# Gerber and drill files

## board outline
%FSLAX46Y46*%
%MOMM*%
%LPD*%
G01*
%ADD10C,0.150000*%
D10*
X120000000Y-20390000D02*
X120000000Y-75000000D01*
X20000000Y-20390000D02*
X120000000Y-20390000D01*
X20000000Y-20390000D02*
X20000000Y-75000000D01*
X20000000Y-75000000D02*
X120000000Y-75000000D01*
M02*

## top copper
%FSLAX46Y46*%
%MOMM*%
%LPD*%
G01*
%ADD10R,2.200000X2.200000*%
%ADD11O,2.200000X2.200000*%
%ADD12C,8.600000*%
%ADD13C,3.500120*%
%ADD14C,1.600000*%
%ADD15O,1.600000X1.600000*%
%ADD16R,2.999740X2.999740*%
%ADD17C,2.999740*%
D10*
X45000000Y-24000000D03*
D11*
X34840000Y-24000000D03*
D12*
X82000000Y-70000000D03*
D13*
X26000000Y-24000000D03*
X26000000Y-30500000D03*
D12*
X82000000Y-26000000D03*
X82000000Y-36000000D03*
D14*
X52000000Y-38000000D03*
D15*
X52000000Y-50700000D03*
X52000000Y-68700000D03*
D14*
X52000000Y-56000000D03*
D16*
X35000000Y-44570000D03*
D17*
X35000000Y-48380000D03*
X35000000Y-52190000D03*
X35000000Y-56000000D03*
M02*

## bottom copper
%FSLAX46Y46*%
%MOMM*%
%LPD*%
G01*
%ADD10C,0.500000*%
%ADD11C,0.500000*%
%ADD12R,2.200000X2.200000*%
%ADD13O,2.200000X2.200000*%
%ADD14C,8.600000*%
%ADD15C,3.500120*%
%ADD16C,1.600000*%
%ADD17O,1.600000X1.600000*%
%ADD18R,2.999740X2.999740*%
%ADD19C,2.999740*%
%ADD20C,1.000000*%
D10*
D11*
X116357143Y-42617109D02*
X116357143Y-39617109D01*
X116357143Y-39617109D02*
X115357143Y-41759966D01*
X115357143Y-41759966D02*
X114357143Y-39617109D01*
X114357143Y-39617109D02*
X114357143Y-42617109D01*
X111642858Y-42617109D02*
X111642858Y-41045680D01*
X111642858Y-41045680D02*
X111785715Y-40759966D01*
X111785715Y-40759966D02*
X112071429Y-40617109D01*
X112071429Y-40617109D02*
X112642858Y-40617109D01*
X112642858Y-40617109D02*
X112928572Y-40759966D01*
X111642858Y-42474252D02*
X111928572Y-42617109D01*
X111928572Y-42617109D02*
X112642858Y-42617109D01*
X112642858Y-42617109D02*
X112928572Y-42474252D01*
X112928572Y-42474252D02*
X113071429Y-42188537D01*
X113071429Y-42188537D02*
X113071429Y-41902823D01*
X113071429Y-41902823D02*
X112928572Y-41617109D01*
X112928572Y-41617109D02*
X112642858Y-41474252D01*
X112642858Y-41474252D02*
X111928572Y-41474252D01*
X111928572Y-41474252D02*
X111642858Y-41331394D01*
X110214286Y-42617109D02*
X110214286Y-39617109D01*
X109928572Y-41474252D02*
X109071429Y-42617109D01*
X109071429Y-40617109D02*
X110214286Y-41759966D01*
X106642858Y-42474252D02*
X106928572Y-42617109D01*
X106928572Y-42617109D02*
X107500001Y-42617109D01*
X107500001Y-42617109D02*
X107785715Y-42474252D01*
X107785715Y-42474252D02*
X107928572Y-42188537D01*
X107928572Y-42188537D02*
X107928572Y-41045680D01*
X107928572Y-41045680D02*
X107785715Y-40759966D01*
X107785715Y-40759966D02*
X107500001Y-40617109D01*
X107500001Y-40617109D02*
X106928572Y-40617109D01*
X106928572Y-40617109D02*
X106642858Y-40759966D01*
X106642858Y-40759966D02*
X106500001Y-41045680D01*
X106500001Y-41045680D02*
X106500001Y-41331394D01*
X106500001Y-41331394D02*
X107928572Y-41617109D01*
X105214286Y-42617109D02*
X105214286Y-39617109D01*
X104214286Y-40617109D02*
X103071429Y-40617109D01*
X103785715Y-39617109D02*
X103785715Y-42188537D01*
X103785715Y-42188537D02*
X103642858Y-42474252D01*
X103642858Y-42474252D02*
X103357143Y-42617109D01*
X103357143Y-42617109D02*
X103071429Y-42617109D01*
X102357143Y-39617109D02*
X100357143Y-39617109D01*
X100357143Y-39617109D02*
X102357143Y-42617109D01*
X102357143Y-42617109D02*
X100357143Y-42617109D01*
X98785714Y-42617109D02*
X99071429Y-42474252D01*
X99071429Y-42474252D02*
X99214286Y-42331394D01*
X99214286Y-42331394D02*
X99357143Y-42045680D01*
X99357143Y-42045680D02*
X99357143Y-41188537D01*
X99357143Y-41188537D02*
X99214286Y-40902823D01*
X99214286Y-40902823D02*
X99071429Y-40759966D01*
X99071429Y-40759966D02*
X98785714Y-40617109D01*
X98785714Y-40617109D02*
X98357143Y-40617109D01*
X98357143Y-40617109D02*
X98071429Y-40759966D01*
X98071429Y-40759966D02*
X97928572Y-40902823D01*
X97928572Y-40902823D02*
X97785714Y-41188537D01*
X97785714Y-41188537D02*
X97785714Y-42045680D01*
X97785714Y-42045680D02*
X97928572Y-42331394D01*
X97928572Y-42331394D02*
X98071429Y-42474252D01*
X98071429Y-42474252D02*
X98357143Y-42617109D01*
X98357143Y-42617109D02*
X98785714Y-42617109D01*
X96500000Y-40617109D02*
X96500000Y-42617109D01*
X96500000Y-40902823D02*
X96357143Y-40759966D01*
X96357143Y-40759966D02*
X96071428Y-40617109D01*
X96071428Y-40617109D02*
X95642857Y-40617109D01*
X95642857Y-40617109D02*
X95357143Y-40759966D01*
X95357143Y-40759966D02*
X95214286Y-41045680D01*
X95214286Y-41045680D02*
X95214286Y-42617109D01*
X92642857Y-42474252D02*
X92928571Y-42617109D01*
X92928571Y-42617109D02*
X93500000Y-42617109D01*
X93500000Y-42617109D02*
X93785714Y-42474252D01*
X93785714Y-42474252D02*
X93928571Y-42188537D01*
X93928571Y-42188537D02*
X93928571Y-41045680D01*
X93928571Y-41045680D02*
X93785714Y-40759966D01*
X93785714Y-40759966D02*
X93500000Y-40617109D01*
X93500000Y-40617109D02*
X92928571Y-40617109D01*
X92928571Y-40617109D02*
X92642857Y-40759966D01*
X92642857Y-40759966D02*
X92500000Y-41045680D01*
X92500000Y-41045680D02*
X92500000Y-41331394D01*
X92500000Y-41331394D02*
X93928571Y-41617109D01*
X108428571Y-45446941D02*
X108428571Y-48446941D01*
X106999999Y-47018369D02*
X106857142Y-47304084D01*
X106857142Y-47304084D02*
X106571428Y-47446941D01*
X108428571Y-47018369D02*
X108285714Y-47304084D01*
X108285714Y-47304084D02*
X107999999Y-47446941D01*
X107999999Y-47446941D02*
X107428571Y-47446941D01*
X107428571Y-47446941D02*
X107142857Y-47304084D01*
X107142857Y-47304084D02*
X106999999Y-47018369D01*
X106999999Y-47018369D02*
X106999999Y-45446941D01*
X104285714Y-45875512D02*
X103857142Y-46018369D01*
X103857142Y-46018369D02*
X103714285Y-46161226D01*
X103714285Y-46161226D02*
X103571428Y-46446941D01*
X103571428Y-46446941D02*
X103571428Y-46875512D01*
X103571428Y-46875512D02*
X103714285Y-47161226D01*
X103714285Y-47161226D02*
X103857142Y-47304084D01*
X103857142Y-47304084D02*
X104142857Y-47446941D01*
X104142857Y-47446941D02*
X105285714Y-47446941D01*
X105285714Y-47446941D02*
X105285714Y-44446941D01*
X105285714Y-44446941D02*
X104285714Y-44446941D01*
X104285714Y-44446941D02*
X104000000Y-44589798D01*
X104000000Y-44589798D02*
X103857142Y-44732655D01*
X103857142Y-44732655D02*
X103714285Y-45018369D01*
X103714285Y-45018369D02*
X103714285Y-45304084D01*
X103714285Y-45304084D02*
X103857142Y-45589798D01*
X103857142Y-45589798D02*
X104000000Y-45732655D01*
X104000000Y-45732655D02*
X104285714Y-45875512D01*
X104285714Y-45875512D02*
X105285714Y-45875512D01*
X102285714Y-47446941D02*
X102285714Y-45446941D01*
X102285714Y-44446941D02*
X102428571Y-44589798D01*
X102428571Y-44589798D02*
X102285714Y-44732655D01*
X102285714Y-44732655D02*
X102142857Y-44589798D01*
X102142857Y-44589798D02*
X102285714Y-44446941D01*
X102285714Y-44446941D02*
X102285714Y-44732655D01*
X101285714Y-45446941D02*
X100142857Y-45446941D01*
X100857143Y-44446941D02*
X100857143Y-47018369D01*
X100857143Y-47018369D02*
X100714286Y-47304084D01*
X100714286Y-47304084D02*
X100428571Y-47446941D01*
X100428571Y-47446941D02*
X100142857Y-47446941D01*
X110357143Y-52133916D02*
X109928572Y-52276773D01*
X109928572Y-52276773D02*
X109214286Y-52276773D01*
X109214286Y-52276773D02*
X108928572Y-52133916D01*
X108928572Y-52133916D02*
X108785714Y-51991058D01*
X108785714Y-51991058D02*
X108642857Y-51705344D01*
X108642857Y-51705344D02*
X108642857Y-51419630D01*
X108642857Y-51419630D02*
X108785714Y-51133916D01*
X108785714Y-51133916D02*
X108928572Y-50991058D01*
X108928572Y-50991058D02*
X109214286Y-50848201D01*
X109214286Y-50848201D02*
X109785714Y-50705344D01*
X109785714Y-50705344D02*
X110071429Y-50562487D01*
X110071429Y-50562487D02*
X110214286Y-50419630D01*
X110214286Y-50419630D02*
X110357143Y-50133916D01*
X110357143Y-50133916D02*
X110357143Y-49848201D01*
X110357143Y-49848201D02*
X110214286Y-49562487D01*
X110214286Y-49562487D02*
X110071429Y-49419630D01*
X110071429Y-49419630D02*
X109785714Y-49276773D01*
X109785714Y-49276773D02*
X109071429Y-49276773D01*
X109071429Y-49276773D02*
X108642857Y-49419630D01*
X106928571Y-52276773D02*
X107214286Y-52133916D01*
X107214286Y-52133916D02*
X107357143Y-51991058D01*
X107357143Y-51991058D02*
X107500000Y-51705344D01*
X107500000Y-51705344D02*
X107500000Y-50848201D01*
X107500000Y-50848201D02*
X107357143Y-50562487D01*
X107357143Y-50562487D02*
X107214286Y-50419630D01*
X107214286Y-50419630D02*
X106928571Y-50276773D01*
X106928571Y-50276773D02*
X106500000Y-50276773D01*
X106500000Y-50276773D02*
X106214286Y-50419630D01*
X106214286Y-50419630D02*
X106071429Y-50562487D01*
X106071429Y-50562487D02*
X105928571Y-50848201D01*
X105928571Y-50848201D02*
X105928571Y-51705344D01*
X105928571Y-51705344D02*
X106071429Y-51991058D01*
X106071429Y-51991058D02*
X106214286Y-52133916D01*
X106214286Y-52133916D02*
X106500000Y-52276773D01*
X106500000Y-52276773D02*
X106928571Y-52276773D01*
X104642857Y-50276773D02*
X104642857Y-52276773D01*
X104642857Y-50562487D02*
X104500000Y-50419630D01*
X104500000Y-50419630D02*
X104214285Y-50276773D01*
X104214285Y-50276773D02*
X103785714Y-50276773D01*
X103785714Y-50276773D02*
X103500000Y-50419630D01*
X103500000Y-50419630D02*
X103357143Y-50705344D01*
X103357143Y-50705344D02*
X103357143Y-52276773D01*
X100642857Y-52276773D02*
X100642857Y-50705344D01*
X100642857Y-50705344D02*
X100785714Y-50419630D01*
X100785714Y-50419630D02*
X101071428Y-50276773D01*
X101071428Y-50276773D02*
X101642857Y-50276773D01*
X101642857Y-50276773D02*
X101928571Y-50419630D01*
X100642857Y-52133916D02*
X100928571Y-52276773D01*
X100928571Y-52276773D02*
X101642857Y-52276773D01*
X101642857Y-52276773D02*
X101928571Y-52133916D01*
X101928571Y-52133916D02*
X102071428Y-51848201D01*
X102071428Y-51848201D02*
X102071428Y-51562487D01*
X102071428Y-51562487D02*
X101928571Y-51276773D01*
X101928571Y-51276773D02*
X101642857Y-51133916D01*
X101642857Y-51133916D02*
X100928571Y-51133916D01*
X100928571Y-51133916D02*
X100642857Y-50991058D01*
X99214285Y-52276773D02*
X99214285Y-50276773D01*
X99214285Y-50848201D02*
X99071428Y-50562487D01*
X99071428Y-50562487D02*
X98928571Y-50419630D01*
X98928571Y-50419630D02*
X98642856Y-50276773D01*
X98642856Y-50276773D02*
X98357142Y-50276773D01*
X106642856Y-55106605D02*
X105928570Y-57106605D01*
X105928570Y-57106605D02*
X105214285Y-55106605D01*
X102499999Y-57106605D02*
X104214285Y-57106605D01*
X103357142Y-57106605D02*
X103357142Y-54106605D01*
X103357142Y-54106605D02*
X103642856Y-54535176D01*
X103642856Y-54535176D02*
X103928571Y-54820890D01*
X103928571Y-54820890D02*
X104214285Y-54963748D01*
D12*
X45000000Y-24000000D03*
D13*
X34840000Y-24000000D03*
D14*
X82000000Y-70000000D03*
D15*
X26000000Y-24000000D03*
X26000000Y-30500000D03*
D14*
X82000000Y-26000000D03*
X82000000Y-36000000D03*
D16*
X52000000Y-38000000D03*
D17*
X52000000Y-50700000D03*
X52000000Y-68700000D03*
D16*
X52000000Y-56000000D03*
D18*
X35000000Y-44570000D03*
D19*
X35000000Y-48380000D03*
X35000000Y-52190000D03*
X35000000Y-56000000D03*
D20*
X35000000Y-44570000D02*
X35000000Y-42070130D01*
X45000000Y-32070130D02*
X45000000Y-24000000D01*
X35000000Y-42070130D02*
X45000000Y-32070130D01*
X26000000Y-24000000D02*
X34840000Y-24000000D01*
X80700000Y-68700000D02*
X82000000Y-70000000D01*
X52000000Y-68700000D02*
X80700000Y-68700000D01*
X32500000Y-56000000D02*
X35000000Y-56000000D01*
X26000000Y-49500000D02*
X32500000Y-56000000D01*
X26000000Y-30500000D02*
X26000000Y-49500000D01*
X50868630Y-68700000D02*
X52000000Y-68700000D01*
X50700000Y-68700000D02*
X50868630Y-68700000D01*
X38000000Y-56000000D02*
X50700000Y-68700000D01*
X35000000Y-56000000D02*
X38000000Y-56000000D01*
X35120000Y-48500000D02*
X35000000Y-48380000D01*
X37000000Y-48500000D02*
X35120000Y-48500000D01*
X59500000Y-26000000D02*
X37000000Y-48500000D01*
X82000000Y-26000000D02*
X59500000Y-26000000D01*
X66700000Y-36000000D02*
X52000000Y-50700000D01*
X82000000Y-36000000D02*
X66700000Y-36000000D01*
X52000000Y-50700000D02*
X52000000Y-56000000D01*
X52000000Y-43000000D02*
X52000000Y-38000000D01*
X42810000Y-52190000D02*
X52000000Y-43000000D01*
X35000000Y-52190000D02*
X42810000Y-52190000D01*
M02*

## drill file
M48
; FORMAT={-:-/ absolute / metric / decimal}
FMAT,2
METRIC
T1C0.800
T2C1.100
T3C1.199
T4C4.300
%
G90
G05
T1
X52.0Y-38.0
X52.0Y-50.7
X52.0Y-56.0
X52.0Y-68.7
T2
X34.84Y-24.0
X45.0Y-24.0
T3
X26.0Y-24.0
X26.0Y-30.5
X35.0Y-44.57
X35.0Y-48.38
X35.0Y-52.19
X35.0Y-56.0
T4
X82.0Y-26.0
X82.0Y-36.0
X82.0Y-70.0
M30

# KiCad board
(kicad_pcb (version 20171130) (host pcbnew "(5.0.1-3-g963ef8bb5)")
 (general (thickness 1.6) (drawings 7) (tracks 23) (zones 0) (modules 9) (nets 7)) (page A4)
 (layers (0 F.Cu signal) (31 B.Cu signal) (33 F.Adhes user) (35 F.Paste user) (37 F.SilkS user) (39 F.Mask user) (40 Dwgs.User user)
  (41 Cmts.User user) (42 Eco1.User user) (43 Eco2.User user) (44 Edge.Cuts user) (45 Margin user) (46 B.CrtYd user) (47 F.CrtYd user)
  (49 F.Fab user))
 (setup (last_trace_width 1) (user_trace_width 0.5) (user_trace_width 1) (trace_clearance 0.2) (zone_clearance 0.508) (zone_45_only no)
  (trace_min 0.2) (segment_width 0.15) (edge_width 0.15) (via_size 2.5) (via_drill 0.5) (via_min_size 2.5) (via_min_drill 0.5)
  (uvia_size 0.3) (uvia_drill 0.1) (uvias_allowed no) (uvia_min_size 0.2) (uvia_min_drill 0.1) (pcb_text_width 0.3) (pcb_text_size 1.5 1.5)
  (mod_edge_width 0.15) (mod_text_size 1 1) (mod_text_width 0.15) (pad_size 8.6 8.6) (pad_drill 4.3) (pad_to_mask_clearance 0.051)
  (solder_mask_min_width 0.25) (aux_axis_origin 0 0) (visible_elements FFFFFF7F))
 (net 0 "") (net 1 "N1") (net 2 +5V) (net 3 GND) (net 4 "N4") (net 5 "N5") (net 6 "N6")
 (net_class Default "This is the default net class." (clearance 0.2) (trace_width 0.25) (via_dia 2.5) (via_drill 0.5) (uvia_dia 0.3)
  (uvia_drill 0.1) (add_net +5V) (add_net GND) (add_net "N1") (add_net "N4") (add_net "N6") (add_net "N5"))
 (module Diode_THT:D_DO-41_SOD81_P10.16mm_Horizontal (layer F.Cu) (at 45 24 180)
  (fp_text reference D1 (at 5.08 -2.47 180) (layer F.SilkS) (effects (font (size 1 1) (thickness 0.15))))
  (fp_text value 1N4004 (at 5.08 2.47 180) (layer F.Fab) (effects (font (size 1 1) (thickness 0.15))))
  (pad 1 thru_hole rect (at 0 0 180) (size 2.2 2.2) (drill 1.1) (layers *.Cu *.Mask) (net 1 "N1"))
  (pad 2 thru_hole oval (at 10.16 0 180) (size 2.2 2.2) (drill 1.1) (layers *.Cu *.Mask) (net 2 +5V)))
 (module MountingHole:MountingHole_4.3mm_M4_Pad (layer F.Cu) (at 82 70)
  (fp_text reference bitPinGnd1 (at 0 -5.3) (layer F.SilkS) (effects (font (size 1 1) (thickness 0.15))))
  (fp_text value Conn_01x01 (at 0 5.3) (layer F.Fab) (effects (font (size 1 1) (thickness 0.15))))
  (pad 1 thru_hole circle (at 0 0) (size 8.6 8.6) (drill 4.3) (layers *.Cu *.Mask) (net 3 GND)))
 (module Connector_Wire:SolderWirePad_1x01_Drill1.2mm (layer F.Cu) (at 26 24 270)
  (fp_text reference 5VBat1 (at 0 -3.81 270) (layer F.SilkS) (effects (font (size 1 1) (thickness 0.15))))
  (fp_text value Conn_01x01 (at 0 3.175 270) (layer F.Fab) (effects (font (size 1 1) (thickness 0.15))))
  (pad 1 thru_hole circle (at 0 0 270) (size 3.50012 3.50012) (drill 1.19888) (layers *.Cu *.Mask) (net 2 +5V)))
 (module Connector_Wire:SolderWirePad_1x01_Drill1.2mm (layer F.Cu) (at 26 30.5 270)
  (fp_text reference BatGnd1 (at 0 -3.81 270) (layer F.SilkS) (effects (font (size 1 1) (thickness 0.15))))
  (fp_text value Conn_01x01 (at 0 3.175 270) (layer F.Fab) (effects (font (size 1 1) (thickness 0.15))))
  (pad 1 thru_hole circle (at 0 0 270) (size 3.50012 3.50012) (drill 1.19888) (layers *.Cu *.Mask) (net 3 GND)))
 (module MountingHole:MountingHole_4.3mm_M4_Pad (layer F.Cu) (at 82 26)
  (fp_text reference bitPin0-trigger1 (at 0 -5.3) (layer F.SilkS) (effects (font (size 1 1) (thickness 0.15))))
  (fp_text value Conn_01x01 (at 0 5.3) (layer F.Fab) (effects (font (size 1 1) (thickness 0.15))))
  (pad 1 thru_hole circle (at 0 0) (size 8.6 8.6) (drill 4.3) (layers *.Cu *.Mask) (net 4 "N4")))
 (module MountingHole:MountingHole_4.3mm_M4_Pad (layer F.Cu) (at 82 36)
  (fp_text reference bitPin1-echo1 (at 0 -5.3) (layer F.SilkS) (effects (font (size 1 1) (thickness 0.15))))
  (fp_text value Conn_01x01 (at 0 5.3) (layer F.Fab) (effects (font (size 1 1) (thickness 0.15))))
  (pad 1 thru_hole circle (at 0 0) (size 8.6 8.6) (drill 4.3) (layers *.Cu *.Mask) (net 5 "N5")))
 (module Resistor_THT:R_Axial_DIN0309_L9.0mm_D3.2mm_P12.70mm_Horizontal (layer F.Cu) (at 52 38 270)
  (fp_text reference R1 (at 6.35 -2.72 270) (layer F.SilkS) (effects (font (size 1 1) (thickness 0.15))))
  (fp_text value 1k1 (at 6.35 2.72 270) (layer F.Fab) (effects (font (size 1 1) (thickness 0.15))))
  (pad 1 thru_hole circle (at 0 0 270) (size 1.6 1.6) (drill 0.8) (layers *.Cu *.Mask) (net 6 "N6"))
  (pad 2 thru_hole oval (at 12.7 0 270) (size 1.6 1.6) (drill 0.8) (layers *.Cu *.Mask) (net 5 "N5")))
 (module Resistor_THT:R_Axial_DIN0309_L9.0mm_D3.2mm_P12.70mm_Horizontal (layer F.Cu) (at 52 56 270)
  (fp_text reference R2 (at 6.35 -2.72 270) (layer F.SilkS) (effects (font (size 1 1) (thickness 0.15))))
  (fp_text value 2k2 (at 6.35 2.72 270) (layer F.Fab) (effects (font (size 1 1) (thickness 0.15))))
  (pad 2 thru_hole oval (at 12.7 0 270) (size 1.6 1.6) (drill 0.8) (layers *.Cu *.Mask) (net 3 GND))
  (pad 1 thru_hole circle (at 0 0 270) (size 1.6 1.6) (drill 0.8) (layers *.Cu *.Mask) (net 5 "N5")))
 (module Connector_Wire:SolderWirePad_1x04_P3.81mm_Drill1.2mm (layer F.Cu) (at 35 44.57 270)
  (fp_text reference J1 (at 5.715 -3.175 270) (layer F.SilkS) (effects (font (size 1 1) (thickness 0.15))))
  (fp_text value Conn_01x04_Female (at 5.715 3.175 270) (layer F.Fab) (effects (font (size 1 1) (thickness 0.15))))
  (pad 1 thru_hole rect (at 0 0 270) (size 2.99974 2.99974) (drill 1.19888) (layers *.Cu *.Mask) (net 1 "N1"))
  (pad 2 thru_hole circle (at 3.81 0 270) (size 2.99974 2.99974) (drill 1.19888) (layers *.Cu *.Mask) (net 4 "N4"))
  (pad 3 thru_hole circle (at 7.62 0 270) (size 2.99974 2.99974) (drill 1.19888) (layers *.Cu *.Mask) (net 6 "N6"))
  (pad 4 thru_hole circle (at 11.43 0 270) (size 2.99974 2.99974) (drill 1.19888) (layers *.Cu *.Mask) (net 3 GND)))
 (gr_line (start 120 20.39) (end 120 75) (layer Edge.Cuts) (width 0.15))
 (gr_line (start 20 20.39) (end 120 20.39) (layer Edge.Cuts) (width 0.15))
 (gr_line (start 20 20.39) (end 20 75) (layer Edge.Cuts) (width 0.15))
 (gr_line (start 20 75) (end 120 75) (layer Edge.Cuts) (width 0.15))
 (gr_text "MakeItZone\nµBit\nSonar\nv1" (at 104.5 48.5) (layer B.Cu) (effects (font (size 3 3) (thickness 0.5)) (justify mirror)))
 (segment (start 35 44.57) (end 35 42.07013) (width 1) (layer B.Cu) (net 1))
 (segment (start 45 32.07013) (end 45 24) (width 1) (layer B.Cu) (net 1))
 (segment (start 35 42.07013) (end 45 32.07013) (width 1) (layer B.Cu) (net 1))
 (segment (start 26 24) (end 34.84 24) (width 1) (layer B.Cu) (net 2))
 (segment (start 80.7 68.7) (end 82 70) (width 1) (layer B.Cu) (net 3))
 (segment (start 52 68.7) (end 80.7 68.7) (width 1) (layer B.Cu) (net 3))
 (segment (start 32.5 56) (end 35 56) (width 1) (layer B.Cu) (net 3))
 (segment (start 26 49.5) (end 32.5 56) (width 1) (layer B.Cu) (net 3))
 (segment (start 26 30.5) (end 26 49.5) (width 1) (layer B.Cu) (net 3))
 (segment (start 50.86863 68.7) (end 52 68.7) (width 1) (layer B.Cu) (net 3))
 (segment (start 50.7 68.7) (end 50.86863 68.7) (width 1) (layer B.Cu) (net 3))
 (segment (start 38 56) (end 50.7 68.7) (width 1) (layer B.Cu) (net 3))
 (segment (start 35 56) (end 38 56) (width 1) (layer B.Cu) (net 3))
 (segment (start 35.12 48.5) (end 35 48.38) (width 1) (layer B.Cu) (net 4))
 (segment (start 37 48.5) (end 35.12 48.5) (width 1) (layer B.Cu) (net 4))
 (segment (start 59.5 26) (end 37 48.5) (width 1) (layer B.Cu) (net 4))
 (segment (start 82 26) (end 59.5 26) (width 1) (layer B.Cu) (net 4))
 (segment (start 66.7 36) (end 52 50.7) (width 1) (layer B.Cu) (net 5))
 (segment (start 82 36) (end 66.7 36) (width 1) (layer B.Cu) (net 5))
 (segment (start 52 50.7) (end 52 56) (width 1) (layer B.Cu) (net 5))
 (segment (start 52 43) (end 52 38) (width 1) (layer B.Cu) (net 6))
 (segment (start 42.81 52.19) (end 52 43) (width 1) (layer B.Cu) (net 6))
 (segment (start 35 52.19) (end 42.81 52.19) (width 1) (layer B.Cu) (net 6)))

